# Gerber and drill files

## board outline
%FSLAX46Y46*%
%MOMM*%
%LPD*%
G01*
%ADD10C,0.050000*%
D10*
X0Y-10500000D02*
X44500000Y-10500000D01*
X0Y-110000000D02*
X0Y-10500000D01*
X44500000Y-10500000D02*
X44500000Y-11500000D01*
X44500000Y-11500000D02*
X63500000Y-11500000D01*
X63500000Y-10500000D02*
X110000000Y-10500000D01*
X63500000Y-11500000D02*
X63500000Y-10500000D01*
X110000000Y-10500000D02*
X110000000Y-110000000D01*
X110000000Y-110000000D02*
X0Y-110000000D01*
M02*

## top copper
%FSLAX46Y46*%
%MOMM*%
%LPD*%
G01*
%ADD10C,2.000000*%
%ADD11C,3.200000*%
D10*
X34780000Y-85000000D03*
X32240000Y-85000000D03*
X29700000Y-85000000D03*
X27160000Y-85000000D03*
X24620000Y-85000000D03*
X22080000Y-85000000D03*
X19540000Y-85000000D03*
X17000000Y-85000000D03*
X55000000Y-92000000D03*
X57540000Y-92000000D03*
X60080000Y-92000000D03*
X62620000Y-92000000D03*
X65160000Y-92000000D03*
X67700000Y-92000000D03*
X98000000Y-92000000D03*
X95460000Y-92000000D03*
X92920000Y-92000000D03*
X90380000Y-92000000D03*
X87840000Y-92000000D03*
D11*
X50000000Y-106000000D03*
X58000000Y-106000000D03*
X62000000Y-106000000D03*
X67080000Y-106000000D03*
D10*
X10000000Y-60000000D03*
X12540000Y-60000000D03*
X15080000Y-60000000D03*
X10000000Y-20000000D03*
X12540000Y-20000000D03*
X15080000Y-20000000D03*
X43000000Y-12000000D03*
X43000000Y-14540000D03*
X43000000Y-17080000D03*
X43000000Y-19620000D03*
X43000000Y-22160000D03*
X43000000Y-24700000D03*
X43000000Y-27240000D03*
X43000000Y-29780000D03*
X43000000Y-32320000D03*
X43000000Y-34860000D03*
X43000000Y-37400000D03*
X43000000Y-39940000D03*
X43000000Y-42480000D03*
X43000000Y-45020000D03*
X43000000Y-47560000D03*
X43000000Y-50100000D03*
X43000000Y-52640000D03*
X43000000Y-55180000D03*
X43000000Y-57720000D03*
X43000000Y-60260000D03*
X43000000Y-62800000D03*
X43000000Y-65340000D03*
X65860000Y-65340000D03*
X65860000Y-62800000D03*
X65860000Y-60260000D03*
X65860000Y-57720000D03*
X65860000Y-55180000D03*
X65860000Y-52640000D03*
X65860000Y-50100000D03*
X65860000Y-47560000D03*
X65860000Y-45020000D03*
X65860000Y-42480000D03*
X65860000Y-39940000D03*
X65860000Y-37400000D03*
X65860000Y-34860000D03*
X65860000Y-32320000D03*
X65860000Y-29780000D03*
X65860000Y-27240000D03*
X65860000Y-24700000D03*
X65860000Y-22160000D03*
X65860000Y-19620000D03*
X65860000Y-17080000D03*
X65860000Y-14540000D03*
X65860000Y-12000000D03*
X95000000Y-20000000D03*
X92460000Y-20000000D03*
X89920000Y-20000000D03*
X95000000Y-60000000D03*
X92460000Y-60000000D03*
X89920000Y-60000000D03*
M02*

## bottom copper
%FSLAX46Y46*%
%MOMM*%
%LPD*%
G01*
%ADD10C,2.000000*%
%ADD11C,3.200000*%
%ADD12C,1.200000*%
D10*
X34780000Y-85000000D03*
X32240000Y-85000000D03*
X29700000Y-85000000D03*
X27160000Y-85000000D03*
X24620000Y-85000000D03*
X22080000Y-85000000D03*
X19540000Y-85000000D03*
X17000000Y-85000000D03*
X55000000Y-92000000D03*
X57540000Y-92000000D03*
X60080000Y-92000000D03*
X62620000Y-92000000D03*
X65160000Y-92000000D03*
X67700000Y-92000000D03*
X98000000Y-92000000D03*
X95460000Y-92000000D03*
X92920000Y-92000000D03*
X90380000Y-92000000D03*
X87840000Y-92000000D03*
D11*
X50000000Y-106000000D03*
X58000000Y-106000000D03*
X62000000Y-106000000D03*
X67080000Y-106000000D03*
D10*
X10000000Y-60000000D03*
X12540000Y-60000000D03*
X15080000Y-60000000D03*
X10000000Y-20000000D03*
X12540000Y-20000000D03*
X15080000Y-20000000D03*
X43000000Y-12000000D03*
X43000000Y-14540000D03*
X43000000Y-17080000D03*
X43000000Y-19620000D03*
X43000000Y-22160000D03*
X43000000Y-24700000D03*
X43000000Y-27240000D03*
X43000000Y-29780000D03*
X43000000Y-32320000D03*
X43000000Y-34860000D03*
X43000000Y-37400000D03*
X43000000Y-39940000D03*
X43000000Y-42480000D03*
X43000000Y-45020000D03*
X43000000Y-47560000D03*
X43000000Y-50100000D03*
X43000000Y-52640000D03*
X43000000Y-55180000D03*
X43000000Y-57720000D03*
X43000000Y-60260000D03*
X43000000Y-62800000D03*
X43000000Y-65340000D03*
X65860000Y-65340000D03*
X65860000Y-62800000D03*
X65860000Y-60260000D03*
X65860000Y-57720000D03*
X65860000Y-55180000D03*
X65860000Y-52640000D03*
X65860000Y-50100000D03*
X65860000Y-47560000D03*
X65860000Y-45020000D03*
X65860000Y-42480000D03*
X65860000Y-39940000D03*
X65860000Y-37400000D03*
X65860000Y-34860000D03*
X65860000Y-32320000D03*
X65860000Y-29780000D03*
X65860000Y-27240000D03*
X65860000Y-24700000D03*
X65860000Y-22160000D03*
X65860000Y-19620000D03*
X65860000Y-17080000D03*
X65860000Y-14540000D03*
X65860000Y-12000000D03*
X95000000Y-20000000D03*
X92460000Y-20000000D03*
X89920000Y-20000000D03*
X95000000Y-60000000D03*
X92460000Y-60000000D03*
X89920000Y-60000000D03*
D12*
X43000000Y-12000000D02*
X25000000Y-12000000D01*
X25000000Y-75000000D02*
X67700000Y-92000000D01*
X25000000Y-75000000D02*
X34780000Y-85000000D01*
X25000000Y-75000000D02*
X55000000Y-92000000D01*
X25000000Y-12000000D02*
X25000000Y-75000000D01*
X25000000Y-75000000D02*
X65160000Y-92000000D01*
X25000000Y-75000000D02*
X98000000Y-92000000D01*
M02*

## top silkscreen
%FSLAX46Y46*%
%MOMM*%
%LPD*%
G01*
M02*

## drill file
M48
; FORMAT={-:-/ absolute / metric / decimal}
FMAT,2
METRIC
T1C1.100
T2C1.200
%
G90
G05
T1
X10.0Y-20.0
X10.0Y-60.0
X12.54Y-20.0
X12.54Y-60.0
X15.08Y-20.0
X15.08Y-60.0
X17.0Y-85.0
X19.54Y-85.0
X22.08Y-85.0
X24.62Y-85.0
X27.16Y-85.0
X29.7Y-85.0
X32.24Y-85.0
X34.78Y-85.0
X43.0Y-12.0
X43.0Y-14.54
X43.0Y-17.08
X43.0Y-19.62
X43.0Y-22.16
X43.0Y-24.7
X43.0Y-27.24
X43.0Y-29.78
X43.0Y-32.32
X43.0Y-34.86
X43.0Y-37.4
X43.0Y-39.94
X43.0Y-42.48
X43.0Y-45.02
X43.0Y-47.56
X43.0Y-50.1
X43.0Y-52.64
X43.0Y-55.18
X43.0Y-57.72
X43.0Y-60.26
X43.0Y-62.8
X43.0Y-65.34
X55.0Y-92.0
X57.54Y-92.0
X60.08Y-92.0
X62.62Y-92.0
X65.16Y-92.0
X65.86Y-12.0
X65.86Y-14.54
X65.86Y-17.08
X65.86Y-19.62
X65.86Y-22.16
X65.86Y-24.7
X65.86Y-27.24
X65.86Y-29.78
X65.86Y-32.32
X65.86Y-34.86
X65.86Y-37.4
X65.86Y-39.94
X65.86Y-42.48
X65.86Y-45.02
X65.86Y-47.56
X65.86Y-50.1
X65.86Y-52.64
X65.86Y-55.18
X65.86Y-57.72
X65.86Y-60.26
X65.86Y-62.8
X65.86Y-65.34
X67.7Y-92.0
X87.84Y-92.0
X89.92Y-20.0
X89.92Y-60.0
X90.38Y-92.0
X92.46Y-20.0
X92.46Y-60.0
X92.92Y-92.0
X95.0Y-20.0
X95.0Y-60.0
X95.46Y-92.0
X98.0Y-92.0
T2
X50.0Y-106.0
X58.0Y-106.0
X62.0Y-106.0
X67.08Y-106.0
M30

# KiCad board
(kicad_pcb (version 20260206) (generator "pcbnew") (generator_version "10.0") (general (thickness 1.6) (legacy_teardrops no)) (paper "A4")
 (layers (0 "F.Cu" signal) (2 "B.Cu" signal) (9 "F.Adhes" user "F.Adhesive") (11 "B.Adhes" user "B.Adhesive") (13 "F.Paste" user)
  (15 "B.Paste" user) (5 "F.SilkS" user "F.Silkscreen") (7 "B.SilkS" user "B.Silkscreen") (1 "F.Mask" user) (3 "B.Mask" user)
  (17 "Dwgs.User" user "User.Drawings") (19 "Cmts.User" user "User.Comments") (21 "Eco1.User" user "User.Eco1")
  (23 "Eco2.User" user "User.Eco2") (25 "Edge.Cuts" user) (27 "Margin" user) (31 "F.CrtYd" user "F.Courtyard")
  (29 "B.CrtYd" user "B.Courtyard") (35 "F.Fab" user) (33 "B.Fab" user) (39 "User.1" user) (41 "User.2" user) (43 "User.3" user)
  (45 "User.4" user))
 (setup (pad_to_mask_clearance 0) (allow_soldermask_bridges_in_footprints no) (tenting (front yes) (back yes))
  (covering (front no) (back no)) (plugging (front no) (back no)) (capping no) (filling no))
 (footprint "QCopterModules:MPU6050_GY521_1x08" (layer "F.Cu") (at 34.78 85 -90)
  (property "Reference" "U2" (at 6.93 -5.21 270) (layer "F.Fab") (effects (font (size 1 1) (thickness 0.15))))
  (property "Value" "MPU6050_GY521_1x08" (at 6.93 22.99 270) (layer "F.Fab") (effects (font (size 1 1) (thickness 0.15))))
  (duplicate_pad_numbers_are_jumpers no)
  (pad "1" thru_hole circle (at 0 0 270) (size 2 2) (drill 1.1) (layers "*.Cu" "*.Mask") (remove_unused_layers no) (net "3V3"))
  (pad "2" thru_hole circle (at 0 2.54 270) (size 2 2) (drill 1.1) (layers "*.Cu" "*.Mask") (remove_unused_layers no) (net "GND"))
  (pad "3" thru_hole circle (at 0 5.08 270) (size 2 2) (drill 1.1) (layers "*.Cu" "*.Mask") (remove_unused_layers no) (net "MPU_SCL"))
  (pad "4" thru_hole circle (at 0 7.62 270) (size 2 2) (drill 1.1) (layers "*.Cu" "*.Mask") (remove_unused_layers no) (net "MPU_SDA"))
  (pad "5" thru_hole circle (at 0 10.16 270) (size 2 2) (drill 1.1) (layers "*.Cu" "*.Mask") (remove_unused_layers no)
   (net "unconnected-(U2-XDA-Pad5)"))
  (pad "6" thru_hole circle (at 0 12.7 270) (size 2 2) (drill 1.1) (layers "*.Cu" "*.Mask") (remove_unused_layers no)
   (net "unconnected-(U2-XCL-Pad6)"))
  (pad "7" thru_hole circle (at 0 15.24 270) (size 2 2) (drill 1.1) (layers "*.Cu" "*.Mask") (remove_unused_layers no) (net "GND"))
  (pad "8" thru_hole circle (at 0 17.78 270) (size 2 2) (drill 1.1) (layers "*.Cu" "*.Mask") (remove_unused_layers no) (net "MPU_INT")))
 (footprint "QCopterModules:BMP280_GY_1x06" (layer "F.Cu") (at 55 92 90)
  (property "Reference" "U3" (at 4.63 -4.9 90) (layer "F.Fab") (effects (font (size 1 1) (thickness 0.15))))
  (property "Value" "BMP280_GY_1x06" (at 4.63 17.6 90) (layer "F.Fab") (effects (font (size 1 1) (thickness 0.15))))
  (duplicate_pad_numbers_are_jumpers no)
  (pad "1" thru_hole circle (at 0 0 90) (size 2 2) (drill 1.1) (layers "*.Cu" "*.Mask") (remove_unused_layers no) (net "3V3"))
  (pad "2" thru_hole circle (at 0 2.54 90) (size 2 2) (drill 1.1) (layers "*.Cu" "*.Mask") (remove_unused_layers no) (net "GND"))
  (pad "3" thru_hole circle (at 0 5.08 90) (size 2 2) (drill 1.1) (layers "*.Cu" "*.Mask") (remove_unused_layers no) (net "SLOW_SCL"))
  (pad "4" thru_hole circle (at 0 7.62 90) (size 2 2) (drill 1.1) (layers "*.Cu" "*.Mask") (remove_unused_layers no) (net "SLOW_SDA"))
  (pad "5" thru_hole circle (at 0 10.16 90) (size 2 2) (drill 1.1) (layers "*.Cu" "*.Mask") (remove_unused_layers no) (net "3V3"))
  (pad "6" thru_hole circle (at 0 12.7 90) (size 2 2) (drill 1.1) (layers "*.Cu" "*.Mask") (remove_unused_layers no) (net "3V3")))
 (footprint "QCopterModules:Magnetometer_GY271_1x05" (layer "F.Cu") (at 98 92 -90)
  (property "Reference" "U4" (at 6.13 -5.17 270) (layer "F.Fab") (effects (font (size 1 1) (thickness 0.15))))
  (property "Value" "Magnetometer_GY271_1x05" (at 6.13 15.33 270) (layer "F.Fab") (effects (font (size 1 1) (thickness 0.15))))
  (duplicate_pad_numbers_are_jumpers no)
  (pad "1" thru_hole circle (at 0 0 270) (size 2 2) (drill 1.1) (layers "*.Cu" "*.Mask") (remove_unused_layers no) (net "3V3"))
  (pad "2" thru_hole circle (at 0 2.54 270) (size 2 2) (drill 1.1) (layers "*.Cu" "*.Mask") (remove_unused_layers no) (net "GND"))
  (pad "3" thru_hole circle (at 0 5.08 270) (size 2 2) (drill 1.1) (layers "*.Cu" "*.Mask") (remove_unused_layers no) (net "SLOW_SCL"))
  (pad "4" thru_hole circle (at 0 7.62 270) (size 2 2) (drill 1.1) (layers "*.Cu" "*.Mask") (remove_unused_layers no) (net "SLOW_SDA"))
  (pad "5" thru_hole circle (at 0 10.16 270) (size 2 2) (drill 1.1) (layers "*.Cu" "*.Mask") (remove_unused_layers no) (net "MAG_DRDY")))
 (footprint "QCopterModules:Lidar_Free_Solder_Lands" (layer "F.Cu") (at 50 106)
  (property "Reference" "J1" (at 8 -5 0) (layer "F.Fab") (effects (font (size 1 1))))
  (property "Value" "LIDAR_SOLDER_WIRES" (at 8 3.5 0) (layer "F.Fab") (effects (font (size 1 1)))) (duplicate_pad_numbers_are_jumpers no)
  (pad "1" thru_hole circle (at 0 0) (size 3.2 3.2) (drill 1.2) (layers "*.Cu" "*.Mask") (remove_unused_layers no) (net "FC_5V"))
  (pad "2" thru_hole circle (at 8 0) (size 3.2 3.2) (drill 1.2) (layers "*.Cu" "*.Mask") (remove_unused_layers no) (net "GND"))
  (pad "3" thru_hole circle (at 12 0) (size 3.2 3.2) (drill 1.2) (layers "*.Cu" "*.Mask") (remove_unused_layers no) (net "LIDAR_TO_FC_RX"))
  (pad "4" thru_hole circle (at 17.08 0) (size 3.2 3.2) (drill 1.2) (layers "*.Cu" "*.Mask") (remove_unused_layers no)
   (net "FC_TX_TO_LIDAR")))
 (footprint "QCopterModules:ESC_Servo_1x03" (layer "F.Cu") (at 10 60 90)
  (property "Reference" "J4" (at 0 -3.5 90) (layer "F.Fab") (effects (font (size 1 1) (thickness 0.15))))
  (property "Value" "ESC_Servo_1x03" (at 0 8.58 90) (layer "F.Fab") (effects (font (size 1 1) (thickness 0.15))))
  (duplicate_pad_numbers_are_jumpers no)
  (pad "1" thru_hole circle (at 0 0 90) (size 2 2) (drill 1.1) (layers "*.Cu" "*.Mask") (remove_unused_layers no) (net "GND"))
  (pad "2" thru_hole circle (at 0 2.54 90) (size 2 2) (drill 1.1) (layers "*.Cu" "*.Mask") (remove_unused_layers no) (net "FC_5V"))
  (pad "3" thru_hole circle (at 0 5.08 90) (size 2 2) (drill 1.1) (layers "*.Cu" "*.Mask") (remove_unused_layers no) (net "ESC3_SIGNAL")))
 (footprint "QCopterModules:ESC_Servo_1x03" (layer "F.Cu") (at 10 20 90)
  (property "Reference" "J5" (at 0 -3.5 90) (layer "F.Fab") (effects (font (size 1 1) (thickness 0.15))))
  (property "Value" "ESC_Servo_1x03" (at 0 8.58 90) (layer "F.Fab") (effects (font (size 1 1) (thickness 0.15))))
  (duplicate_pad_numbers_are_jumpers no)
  (pad "1" thru_hole circle (at 0 0 90) (size 2 2) (drill 1.1) (layers "*.Cu" "*.Mask") (remove_unused_layers no) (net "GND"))
  (pad "2" thru_hole circle (at 0 2.54 90) (size 2 2) (drill 1.1) (layers "*.Cu" "*.Mask") (remove_unused_layers no)
   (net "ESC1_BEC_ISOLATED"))
  (pad "3" thru_hole circle (at 0 5.08 90) (size 2 2) (drill 1.1) (layers "*.Cu" "*.Mask") (remove_unused_layers no) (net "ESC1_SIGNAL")))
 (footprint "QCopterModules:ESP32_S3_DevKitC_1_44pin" (layer "F.Cu") (at 43 12)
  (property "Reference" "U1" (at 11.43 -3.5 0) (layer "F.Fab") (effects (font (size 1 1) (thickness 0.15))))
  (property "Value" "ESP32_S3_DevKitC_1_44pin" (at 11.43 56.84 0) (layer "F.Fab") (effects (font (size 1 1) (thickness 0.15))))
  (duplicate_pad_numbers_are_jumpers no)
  (pad "1" thru_hole circle (at 0 0) (size 2 2) (drill 1.1) (layers "*.Cu" "*.Mask") (remove_unused_layers no) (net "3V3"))
  (pad "2" thru_hole circle (at 0 2.54) (size 2 2) (drill 1.1) (layers "*.Cu" "*.Mask") (remove_unused_layers no))
  (pad "3" thru_hole circle (at 0 5.08) (size 2 2) (drill 1.1) (layers "*.Cu" "*.Mask") (remove_unused_layers no)
   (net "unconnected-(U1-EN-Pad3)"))
  (pad "4" thru_hole circle (at 0 7.62) (size 2 2) (drill 1.1) (layers "*.Cu" "*.Mask") (remove_unused_layers no) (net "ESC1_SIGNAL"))
  (pad "5" thru_hole circle (at 0 10.16) (size 2 2) (drill 1.1) (layers "*.Cu" "*.Mask") (remove_unused_layers no)
   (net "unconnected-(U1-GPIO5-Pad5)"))
  (pad "6" thru_hole circle (at 0 12.7) (size 2 2) (drill 1.1) (layers "*.Cu" "*.Mask") (remove_unused_layers no)
   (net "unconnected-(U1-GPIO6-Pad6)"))
  (pad "7" thru_hole circle (at 0 15.24) (size 2 2) (drill 1.1) (layers "*.Cu" "*.Mask") (remove_unused_layers no)
   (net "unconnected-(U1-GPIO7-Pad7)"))
  (pad "8" thru_hole circle (at 0 17.78) (size 2 2) (drill 1.1) (layers "*.Cu" "*.Mask") (remove_unused_layers no) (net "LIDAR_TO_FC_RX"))
  (pad "9" thru_hole circle (at 0 20.32) (size 2 2) (drill 1.1) (layers "*.Cu" "*.Mask") (remove_unused_layers no) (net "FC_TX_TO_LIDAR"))
  (pad "10" thru_hole circle (at 0 22.86) (size 2 2) (drill 1.1) (layers "*.Cu" "*.Mask") (remove_unused_layers no)
   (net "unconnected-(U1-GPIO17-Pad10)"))
  (pad "11" thru_hole circle (at 0 25.4) (size 2 2) (drill 1.1) (layers "*.Cu" "*.Mask") (remove_unused_layers no) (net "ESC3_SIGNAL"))
  (pad "12" thru_hole circle (at 0 27.94) (size 2 2) (drill 1.1) (layers "*.Cu" "*.Mask") (remove_unused_layers no)
   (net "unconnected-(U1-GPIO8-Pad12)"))
  (pad "13" thru_hole circle (at 0 30.48) (size 2 2) (drill 1.1) (layers "*.Cu" "*.Mask") (remove_unused_layers no)
   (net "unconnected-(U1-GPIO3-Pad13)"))
  (pad "14" thru_hole circle (at 0 33.02) (size 2 2) (drill 1.1) (layers "*.Cu" "*.Mask") (remove_unused_layers no)
   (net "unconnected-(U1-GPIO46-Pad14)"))
  (pad "15" thru_hole circle (at 0 35.56) (size 2 2) (drill 1.1) (layers "*.Cu" "*.Mask") (remove_unused_layers no)
   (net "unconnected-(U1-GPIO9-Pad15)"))
  (pad "16" thru_hole circle (at 0 38.1) (size 2 2) (drill 1.1) (layers "*.Cu" "*.Mask") (remove_unused_layers no)
   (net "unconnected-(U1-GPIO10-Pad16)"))
  (pad "17" thru_hole circle (at 0 40.64) (size 2 2) (drill 1.1) (layers "*.Cu" "*.Mask") (remove_unused_layers no)
   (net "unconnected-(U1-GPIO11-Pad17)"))
  (pad "18" thru_hole circle (at 0 43.18) (size 2 2) (drill 1.1) (layers "*.Cu" "*.Mask") (remove_unused_layers no) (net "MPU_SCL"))
  (pad "19" thru_hole circle (at 0 45.72) (size 2 2) (drill 1.1) (layers "*.Cu" "*.Mask") (remove_unused_layers no) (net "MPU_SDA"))
  (pad "20" thru_hole circle (at 0 48.26) (size 2 2) (drill 1.1) (layers "*.Cu" "*.Mask") (remove_unused_layers no) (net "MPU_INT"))
  (pad "21" thru_hole circle (at 0 50.8) (size 2 2) (drill 1.1) (layers "*.Cu" "*.Mask") (remove_unused_layers no) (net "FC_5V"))
  (pad "22" thru_hole circle (at 0 53.34) (size 2 2) (drill 1.1) (layers "*.Cu" "*.Mask") (remove_unused_layers no) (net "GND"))
  (pad "23" thru_hole circle (at 22.86 53.34) (size 2 2) (drill 1.1) (layers "*.Cu" "*.Mask") (remove_unused_layers no) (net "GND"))
  (pad "24" thru_hole circle (at 22.86 50.8) (size 2 2) (drill 1.1) (layers "*.Cu" "*.Mask") (remove_unused_layers no) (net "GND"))
  (pad "25" thru_hole circle (at 22.86 48.26) (size 2 2) (drill 1.1) (layers "*.Cu" "*.Mask") (remove_unused_layers no)
   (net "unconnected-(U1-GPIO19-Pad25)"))
  (pad "26" thru_hole circle (at 22.86 45.72) (size 2 2) (drill 1.1) (layers "*.Cu" "*.Mask") (remove_unused_layers no)
   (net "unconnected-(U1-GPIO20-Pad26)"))
  (pad "27" thru_hole circle (at 22.86 43.18) (size 2 2) (drill 1.1) (layers "*.Cu" "*.Mask") (remove_unused_layers no) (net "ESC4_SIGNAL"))
  (pad "28" thru_hole circle (at 22.86 40.64) (size 2 2) (drill 1.1) (layers "*.Cu" "*.Mask") (remove_unused_layers no)
   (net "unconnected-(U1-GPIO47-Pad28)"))
  (pad "29" thru_hole circle (at 22.86 38.1) (size 2 2) (drill 1.1) (layers "*.Cu" "*.Mask") (remove_unused_layers no)
   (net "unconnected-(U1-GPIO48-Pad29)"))
  (pad "30" thru_hole circle (at 22.86 35.56) (size 2 2) (drill 1.1) (layers "*.Cu" "*.Mask") (remove_unused_layers no)
   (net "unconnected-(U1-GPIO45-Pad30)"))
  (pad "31" thru_hole circle (at 22.86 33.02) (size 2 2) (drill 1.1) (layers "*.Cu" "*.Mask") (remove_unused_layers no)
   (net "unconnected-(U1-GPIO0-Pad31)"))
  (pad "32" thru_hole circle (at 22.86 30.48) (size 2 2) (drill 1.1) (layers "*.Cu" "*.Mask") (remove_unused_layers no)
   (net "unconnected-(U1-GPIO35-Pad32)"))
  (pad "33" thru_hole circle (at 22.86 27.94) (size 2 2) (drill 1.1) (layers "*.Cu" "*.Mask") (remove_unused_layers no)
   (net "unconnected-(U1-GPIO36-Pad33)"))
  (pad "34" thru_hole circle (at 22.86 25.4) (size 2 2) (drill 1.1) (layers "*.Cu" "*.Mask") (remove_unused_layers no)
   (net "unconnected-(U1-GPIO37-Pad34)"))
  (pad "35" thru_hole circle (at 22.86 22.86) (size 2 2) (drill 1.1) (layers "*.Cu" "*.Mask") (remove_unused_layers no)
   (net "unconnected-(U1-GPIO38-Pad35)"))
  (pad "36" thru_hole circle (at 22.86 20.32) (size 2 2) (drill 1.1) (layers "*.Cu" "*.Mask") (remove_unused_layers no) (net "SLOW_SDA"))
  (pad "37" thru_hole circle (at 22.86 17.78) (size 2 2) (drill 1.1) (layers "*.Cu" "*.Mask") (remove_unused_layers no) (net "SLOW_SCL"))
  (pad "38" thru_hole circle (at 22.86 15.24) (size 2 2) (drill 1.1) (layers "*.Cu" "*.Mask") (remove_unused_layers no) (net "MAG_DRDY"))
  (pad "39" thru_hole circle (at 22.86 12.7) (size 2 2) (drill 1.1) (layers "*.Cu" "*.Mask") (remove_unused_layers no)
   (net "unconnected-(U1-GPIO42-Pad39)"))
  (pad "40" thru_hole circle (at 22.86 10.16) (size 2 2) (drill 1.1) (layers "*.Cu" "*.Mask") (remove_unused_layers no) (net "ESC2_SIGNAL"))
  (pad "41" thru_hole circle (at 22.86 7.62) (size 2 2) (drill 1.1) (layers "*.Cu" "*.Mask") (remove_unused_layers no)
   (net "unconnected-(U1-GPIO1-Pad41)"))
  (pad "42" thru_hole circle (at 22.86 5.08) (size 2 2) (drill 1.1) (layers "*.Cu" "*.Mask") (remove_unused_layers no)
   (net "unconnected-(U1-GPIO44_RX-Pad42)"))
  (pad "43" thru_hole circle (at 22.86 2.54) (size 2 2) (drill 1.1) (layers "*.Cu" "*.Mask") (remove_unused_layers no)
   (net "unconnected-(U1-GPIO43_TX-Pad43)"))
  (pad "44" thru_hole circle (at 22.86 0) (size 2 2) (drill 1.1) (layers "*.Cu" "*.Mask") (remove_unused_layers no) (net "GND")))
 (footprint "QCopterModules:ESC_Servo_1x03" (layer "F.Cu") (at 95 20 -90)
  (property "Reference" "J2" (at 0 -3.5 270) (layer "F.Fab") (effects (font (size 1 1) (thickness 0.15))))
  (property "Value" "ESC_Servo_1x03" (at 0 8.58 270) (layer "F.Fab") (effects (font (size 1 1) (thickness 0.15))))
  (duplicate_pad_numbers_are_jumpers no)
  (pad "1" thru_hole circle (at 0 0 270) (size 2 2) (drill 1.1) (layers "*.Cu" "*.Mask") (remove_unused_layers no) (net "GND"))
  (pad "2" thru_hole circle (at 0 2.54 270) (size 2 2) (drill 1.1) (layers "*.Cu" "*.Mask") (remove_unused_layers no)
   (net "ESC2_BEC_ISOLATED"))
  (pad "3" thru_hole circle (at 0 5.08 270) (size 2 2) (drill 1.1) (layers "*.Cu" "*.Mask") (remove_unused_layers no) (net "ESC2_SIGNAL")))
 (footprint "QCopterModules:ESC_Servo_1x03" (layer "F.Cu") (at 95 60 -90)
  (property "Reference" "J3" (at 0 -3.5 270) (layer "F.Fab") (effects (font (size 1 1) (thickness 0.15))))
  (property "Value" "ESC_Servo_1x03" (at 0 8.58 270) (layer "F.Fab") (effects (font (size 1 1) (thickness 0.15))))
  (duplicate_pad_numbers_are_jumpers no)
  (pad "1" thru_hole circle (at 0 0 270) (size 2 2) (drill 1.1) (layers "*.Cu" "*.Mask") (remove_unused_layers no) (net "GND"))
  (pad "2" thru_hole circle (at 0 2.54 270) (size 2 2) (drill 1.1) (layers "*.Cu" "*.Mask") (remove_unused_layers no)
   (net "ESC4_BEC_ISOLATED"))
  (pad "3" thru_hole circle (at 0 5.08 270) (size 2 2) (drill 1.1) (layers "*.Cu" "*.Mask") (remove_unused_layers no) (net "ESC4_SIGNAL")))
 (gr_line (start 0 10.5) (end 44.5 10.5) (stroke (width 0.05) (type default)) (layer "Edge.Cuts"))
 (gr_line (start 0 110) (end 0 10.5) (stroke (width 0.05) (type default)) (layer "Edge.Cuts"))
 (gr_line (start 44.5 10.5) (end 44.5 11.5) (stroke (width 0.05) (type default)) (layer "Edge.Cuts"))
 (gr_line (start 44.5 11.5) (end 63.5 11.5) (stroke (width 0.05) (type default)) (layer "Edge.Cuts"))
 (gr_line (start 63.5 10.5) (end 110 10.5) (stroke (width 0.05) (type default)) (layer "Edge.Cuts"))
 (gr_line (start 63.5 11.5) (end 63.5 10.5) (stroke (width 0.05) (type default)) (layer "Edge.Cuts"))
 (gr_line (start 110 10.5) (end 110 110) (stroke (width 0.05) (type default)) (layer "Edge.Cuts"))
 (gr_line (start 110 110) (end 0 110) (stroke (width 0.05) (type default)) (layer "Edge.Cuts"))
 (segment (start 43 12) (end 25 12) (width 1.2) (layer "B.Cu") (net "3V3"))
 (segment (start 25 75) (end 67.7 92) (width 1.2) (layer "B.Cu") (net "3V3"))
 (segment (start 25 75) (end 34.78 85) (width 1.2) (layer "B.Cu") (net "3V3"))
 (segment (start 25 75) (end 55 92) (width 1.2) (layer "B.Cu") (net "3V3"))
 (segment (start 25 12) (end 25 75) (width 1.2) (layer "B.Cu") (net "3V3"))
 (segment (start 25 75) (end 65.16 92) (width 1.2) (layer "B.Cu") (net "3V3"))
 (segment (start 25 75) (end 98 92) (width 1.2) (layer "B.Cu") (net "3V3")))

